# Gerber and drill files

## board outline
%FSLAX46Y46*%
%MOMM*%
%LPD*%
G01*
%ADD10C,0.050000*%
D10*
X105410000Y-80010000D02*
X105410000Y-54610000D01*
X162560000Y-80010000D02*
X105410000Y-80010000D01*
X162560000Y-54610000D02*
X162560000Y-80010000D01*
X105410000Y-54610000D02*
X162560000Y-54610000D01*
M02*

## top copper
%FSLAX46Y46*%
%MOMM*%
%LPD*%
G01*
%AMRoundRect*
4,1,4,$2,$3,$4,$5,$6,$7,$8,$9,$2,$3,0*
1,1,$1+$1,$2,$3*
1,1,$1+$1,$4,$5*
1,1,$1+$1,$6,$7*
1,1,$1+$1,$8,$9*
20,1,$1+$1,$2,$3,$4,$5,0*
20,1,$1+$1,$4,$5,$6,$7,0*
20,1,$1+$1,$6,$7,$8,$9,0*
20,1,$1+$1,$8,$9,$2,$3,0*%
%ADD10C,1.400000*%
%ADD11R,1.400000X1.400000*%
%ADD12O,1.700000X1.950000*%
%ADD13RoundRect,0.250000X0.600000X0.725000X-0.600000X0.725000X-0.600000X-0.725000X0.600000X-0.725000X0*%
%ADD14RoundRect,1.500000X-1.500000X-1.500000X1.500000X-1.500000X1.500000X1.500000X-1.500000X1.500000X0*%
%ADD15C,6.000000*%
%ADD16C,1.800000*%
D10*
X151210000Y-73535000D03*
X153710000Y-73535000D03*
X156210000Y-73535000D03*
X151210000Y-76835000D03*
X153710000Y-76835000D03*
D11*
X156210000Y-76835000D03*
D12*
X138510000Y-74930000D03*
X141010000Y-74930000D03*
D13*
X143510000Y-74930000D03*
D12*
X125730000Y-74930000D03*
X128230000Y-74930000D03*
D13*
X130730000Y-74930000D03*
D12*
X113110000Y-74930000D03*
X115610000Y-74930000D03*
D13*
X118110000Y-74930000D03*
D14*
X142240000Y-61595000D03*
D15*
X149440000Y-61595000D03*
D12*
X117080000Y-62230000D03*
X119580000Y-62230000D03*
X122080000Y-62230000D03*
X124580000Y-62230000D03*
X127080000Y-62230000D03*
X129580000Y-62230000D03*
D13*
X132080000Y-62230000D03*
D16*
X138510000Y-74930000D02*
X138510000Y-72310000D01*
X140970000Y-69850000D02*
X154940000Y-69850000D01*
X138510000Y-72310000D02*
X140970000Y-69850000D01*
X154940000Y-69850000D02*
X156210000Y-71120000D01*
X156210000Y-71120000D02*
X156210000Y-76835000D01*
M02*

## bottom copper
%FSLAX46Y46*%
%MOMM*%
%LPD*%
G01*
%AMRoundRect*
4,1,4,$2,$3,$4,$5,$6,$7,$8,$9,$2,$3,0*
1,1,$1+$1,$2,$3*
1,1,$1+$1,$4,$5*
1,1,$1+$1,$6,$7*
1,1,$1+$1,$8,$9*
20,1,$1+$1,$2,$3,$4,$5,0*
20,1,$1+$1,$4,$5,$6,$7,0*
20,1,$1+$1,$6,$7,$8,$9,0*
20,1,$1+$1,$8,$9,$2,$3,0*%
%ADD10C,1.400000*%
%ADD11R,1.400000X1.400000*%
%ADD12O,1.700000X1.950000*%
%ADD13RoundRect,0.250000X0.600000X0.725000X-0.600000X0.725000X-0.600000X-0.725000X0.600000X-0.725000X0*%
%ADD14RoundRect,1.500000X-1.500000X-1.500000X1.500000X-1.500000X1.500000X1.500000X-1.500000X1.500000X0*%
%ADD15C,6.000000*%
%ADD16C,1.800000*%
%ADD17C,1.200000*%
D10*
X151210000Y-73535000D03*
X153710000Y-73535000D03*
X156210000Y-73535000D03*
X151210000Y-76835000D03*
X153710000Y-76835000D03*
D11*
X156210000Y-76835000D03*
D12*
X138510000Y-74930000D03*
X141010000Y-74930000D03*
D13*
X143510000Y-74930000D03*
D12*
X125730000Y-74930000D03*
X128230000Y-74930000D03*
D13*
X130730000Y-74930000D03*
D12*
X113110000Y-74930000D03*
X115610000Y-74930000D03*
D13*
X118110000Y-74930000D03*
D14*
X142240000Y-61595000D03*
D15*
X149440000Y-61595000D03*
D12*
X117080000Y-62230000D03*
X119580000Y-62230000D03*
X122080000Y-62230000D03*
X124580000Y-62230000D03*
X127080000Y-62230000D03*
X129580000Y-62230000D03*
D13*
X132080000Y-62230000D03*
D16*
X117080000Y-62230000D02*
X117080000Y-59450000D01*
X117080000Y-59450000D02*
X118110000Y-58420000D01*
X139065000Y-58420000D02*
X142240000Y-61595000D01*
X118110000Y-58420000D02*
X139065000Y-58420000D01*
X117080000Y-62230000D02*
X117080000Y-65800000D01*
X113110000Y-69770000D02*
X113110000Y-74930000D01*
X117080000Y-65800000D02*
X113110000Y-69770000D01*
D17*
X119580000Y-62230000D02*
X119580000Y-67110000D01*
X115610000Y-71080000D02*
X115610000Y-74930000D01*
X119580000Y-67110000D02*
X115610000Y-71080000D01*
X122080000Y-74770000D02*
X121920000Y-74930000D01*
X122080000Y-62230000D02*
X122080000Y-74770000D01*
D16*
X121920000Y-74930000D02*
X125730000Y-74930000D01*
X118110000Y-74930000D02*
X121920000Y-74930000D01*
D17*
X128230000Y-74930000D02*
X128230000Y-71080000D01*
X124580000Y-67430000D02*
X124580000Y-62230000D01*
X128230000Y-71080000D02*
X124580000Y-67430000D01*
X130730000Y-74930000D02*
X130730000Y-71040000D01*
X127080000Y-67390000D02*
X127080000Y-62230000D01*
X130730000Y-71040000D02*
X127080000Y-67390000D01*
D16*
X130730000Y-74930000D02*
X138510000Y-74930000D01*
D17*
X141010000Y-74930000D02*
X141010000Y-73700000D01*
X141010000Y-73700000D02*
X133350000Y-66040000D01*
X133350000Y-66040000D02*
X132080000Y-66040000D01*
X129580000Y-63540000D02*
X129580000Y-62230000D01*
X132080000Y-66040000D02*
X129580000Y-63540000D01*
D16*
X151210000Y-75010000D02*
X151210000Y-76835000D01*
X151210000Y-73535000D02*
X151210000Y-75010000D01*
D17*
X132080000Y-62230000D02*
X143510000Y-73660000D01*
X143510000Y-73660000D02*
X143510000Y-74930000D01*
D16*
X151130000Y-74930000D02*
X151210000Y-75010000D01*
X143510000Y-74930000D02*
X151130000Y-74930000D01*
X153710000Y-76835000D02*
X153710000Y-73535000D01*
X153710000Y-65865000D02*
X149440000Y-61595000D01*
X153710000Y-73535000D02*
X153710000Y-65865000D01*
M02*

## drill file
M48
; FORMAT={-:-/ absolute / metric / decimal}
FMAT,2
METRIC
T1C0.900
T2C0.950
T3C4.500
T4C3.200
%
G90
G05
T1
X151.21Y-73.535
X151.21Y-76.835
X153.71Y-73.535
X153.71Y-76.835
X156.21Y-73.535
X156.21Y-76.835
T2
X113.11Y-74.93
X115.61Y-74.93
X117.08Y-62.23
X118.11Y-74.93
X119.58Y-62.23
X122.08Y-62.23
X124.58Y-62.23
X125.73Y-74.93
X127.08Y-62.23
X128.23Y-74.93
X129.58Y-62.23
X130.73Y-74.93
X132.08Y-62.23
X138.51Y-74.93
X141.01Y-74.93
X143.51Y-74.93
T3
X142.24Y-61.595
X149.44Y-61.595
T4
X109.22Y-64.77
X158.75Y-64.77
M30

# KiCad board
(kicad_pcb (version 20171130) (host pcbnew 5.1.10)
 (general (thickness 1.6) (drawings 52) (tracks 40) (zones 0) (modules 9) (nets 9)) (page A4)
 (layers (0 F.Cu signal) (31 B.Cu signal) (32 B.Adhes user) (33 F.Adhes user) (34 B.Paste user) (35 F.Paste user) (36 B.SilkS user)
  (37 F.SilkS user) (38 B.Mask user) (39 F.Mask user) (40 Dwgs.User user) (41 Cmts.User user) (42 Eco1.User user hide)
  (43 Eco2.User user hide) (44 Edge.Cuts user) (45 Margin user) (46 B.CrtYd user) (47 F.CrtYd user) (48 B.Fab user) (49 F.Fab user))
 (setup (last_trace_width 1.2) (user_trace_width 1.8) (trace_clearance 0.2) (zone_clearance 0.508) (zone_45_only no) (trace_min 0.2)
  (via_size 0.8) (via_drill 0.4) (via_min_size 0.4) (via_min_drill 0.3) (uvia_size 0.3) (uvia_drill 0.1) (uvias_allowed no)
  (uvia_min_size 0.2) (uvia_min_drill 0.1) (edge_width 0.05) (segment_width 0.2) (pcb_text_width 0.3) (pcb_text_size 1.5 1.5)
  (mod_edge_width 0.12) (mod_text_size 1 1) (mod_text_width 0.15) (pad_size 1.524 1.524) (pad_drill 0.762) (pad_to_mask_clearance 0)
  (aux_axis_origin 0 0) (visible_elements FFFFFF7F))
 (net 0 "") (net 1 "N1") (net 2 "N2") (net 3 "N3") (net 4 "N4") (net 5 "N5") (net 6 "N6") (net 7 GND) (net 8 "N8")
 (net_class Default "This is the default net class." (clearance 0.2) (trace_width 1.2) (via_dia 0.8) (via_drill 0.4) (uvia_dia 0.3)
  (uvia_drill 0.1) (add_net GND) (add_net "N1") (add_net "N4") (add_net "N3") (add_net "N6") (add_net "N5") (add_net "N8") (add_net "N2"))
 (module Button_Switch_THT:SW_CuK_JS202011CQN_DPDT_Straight (layer F.Cu) (at 156.21 76.835 180)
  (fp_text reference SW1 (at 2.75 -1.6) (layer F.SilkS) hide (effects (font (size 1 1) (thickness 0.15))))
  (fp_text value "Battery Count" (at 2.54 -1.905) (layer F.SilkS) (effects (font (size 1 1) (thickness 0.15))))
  (pad 6 thru_hole circle (at 5 3.3 180) (size 1.4 1.4) (drill 0.9) (layers *.Cu *.Mask) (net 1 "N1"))
  (pad 5 thru_hole circle (at 2.5 3.3 180) (size 1.4 1.4) (drill 0.9) (layers *.Cu *.Mask) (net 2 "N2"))
  (pad 4 thru_hole circle (at 0 3.3 180) (size 1.4 1.4) (drill 0.9) (layers *.Cu *.Mask) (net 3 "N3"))
  (pad 3 thru_hole circle (at 5 0 180) (size 1.4 1.4) (drill 0.9) (layers *.Cu *.Mask) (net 1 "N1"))
  (pad 2 thru_hole circle (at 2.5 0 180) (size 1.4 1.4) (drill 0.9) (layers *.Cu *.Mask) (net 2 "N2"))
  (pad 1 thru_hole rect (at 0 0 180) (size 1.4 1.4) (drill 0.9) (layers *.Cu *.Mask) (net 3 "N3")))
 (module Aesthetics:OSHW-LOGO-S (layer F.Cu) (at 109.22 58.42)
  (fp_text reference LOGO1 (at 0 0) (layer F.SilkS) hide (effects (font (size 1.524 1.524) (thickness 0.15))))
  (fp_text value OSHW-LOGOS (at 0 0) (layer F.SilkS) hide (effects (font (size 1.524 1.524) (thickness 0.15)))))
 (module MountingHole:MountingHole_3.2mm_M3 (layer F.Cu) (at 158.75 64.77)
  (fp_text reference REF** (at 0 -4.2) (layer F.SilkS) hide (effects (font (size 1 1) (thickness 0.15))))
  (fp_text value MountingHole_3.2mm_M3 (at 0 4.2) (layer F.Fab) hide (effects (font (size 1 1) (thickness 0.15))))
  (pad 1 np_thru_hole circle (at 0 0) (size 3.2 3.2) (drill 3.2) (layers *.Cu *.Mask)))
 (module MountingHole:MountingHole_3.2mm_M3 (layer F.Cu) (at 109.22 64.77)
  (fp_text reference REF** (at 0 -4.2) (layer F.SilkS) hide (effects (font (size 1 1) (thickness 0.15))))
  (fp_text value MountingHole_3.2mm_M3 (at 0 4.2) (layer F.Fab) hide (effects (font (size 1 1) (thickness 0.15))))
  (pad 1 np_thru_hole circle (at 0 0) (size 3.2 3.2) (drill 3.2) (layers *.Cu *.Mask)))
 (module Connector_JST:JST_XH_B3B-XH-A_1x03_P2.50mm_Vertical (layer F.Cu) (at 143.51 74.93 180)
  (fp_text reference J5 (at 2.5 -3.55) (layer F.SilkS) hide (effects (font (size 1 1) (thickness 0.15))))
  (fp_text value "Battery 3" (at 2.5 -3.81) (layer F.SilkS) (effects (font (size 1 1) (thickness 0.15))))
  (pad 3 thru_hole oval (at 5 0 180) (size 1.7 1.95) (drill 0.95) (layers *.Cu *.Mask) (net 3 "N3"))
  (pad 2 thru_hole oval (at 2.5 0 180) (size 1.7 1.95) (drill 0.95) (layers *.Cu *.Mask) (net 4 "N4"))
  (pad 1 thru_hole roundrect (at 0 0 180) (size 1.7 1.95) (drill 0.95) (layers *.Cu *.Mask) (roundrect_rratio 0.1470588235294118)
   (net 1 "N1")))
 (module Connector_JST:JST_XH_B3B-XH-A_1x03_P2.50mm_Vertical (layer F.Cu) (at 130.73 74.93 180)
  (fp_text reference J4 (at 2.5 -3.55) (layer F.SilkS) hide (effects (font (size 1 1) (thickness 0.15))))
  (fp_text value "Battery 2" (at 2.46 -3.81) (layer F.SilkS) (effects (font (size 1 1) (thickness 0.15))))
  (pad 3 thru_hole oval (at 5 0 180) (size 1.7 1.95) (drill 0.95) (layers *.Cu *.Mask) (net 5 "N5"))
  (pad 2 thru_hole oval (at 2.5 0 180) (size 1.7 1.95) (drill 0.95) (layers *.Cu *.Mask) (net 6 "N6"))
  (pad 1 thru_hole roundrect (at 0 0 180) (size 1.7 1.95) (drill 0.95) (layers *.Cu *.Mask) (roundrect_rratio 0.1470588235294118)
   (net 3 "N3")))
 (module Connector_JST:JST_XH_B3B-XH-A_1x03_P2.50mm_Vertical (layer F.Cu) (at 118.11 74.93 180)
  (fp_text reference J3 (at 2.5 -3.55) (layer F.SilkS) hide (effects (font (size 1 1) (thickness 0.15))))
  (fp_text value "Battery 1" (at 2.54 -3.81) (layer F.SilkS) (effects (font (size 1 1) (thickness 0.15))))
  (pad 3 thru_hole oval (at 5 0 180) (size 1.7 1.95) (drill 0.95) (layers *.Cu *.Mask) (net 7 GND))
  (pad 2 thru_hole oval (at 2.5 0 180) (size 1.7 1.95) (drill 0.95) (layers *.Cu *.Mask) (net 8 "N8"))
  (pad 1 thru_hole roundrect (at 0 0 180) (size 1.7 1.95) (drill 0.95) (layers *.Cu *.Mask) (roundrect_rratio 0.1470588235294118)
   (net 5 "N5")))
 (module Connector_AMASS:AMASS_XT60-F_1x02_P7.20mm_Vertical (layer F.Cu) (at 142.24 61.595)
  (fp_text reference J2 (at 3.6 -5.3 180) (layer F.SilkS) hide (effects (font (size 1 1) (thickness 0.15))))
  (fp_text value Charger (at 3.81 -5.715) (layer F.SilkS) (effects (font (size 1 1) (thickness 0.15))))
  (pad 1 thru_hole roundrect (at 0 0) (size 6 6) (drill 4.5) (layers *.Cu *.Mask) (roundrect_rratio 0.25) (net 7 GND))
  (pad 2 thru_hole circle (at 7.2 0) (size 6 6) (drill 4.5) (layers *.Cu *.Mask) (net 2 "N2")))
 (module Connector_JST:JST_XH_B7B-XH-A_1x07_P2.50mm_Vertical (layer F.Cu) (at 132.08 62.23 180)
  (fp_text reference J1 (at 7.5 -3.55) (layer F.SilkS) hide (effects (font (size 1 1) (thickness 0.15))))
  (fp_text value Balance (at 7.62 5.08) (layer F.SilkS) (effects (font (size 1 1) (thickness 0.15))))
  (pad 7 thru_hole oval (at 15 0 180) (size 1.7 1.95) (drill 0.95) (layers *.Cu *.Mask) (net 7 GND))
  (pad 6 thru_hole oval (at 12.5 0 180) (size 1.7 1.95) (drill 0.95) (layers *.Cu *.Mask) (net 8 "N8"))
  (pad 5 thru_hole oval (at 10 0 180) (size 1.7 1.95) (drill 0.95) (layers *.Cu *.Mask) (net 5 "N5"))
  (pad 4 thru_hole oval (at 7.5 0 180) (size 1.7 1.95) (drill 0.95) (layers *.Cu *.Mask) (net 6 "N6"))
  (pad 3 thru_hole oval (at 5 0 180) (size 1.7 1.95) (drill 0.95) (layers *.Cu *.Mask) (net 3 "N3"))
  (pad 2 thru_hole oval (at 2.5 0 180) (size 1.7 1.95) (drill 0.95) (layers *.Cu *.Mask) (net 4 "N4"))
  (pad 1 thru_hole roundrect (at 0 0 180) (size 1.7 1.95) (drill 0.95) (layers *.Cu *.Mask) (roundrect_rratio 0.1470588235294118)
   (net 1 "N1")))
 (gr_line (start 105.41 80.01) (end 105.41 54.61) (layer Edge.Cuts) (width 0.05))
 (gr_line (start 162.56 80.01) (end 105.41 80.01) (layer Edge.Cuts) (width 0.05))
 (gr_line (start 162.56 54.61) (end 162.56 80.01) (layer Edge.Cuts) (width 0.05))
 (gr_line (start 105.41 54.61) (end 162.56 54.61) (layer Edge.Cuts) (width 0.05))
 (segment (start 117.08 62.23) (end 117.08 59.45) (width 1.8) (layer B.Cu) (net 7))
 (segment (start 117.08 59.45) (end 118.11 58.42) (width 1.8) (layer B.Cu) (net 7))
 (segment (start 139.065 58.42) (end 142.24 61.595) (width 1.8) (layer B.Cu) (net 7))
 (segment (start 118.11 58.42) (end 139.065 58.42) (width 1.8) (layer B.Cu) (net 7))
 (segment (start 117.08 62.23) (end 117.08 65.8) (width 1.8) (layer B.Cu) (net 7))
 (segment (start 113.11 69.77) (end 113.11 74.93) (width 1.8) (layer B.Cu) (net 7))
 (segment (start 117.08 65.8) (end 113.11 69.77) (width 1.8) (layer B.Cu) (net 7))
 (segment (start 119.58 62.23) (end 119.58 67.11) (width 1.2) (layer B.Cu) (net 8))
 (segment (start 115.61 71.08) (end 115.61 74.93) (width 1.2) (layer B.Cu) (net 8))
 (segment (start 119.58 67.11) (end 115.61 71.08) (width 1.2) (layer B.Cu) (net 8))
 (segment (start 122.08 74.77) (end 121.92 74.93) (width 1.2) (layer B.Cu) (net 5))
 (segment (start 122.08 62.23) (end 122.08 74.77) (width 1.2) (layer B.Cu) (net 5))
 (segment (start 121.92 74.93) (end 125.73 74.93) (width 1.8) (layer B.Cu) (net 5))
 (segment (start 118.11 74.93) (end 121.92 74.93) (width 1.8) (layer B.Cu) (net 5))
 (segment (start 128.23 74.93) (end 128.23 71.08) (width 1.2) (layer B.Cu) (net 6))
 (segment (start 124.58 67.43) (end 124.58 62.23) (width 1.2) (layer B.Cu) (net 6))
 (segment (start 128.23 71.08) (end 124.58 67.43) (width 1.2) (layer B.Cu) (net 6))
 (segment (start 130.73 74.93) (end 130.73 71.04) (width 1.2) (layer B.Cu) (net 3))
 (segment (start 127.08 67.39) (end 127.08 62.23) (width 1.2) (layer B.Cu) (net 3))
 (segment (start 130.73 71.04) (end 127.08 67.39) (width 1.2) (layer B.Cu) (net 3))
 (segment (start 130.73 74.93) (end 138.51 74.93) (width 1.8) (layer B.Cu) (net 3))
 (segment (start 138.51 74.93) (end 138.51 72.31) (width 1.8) (layer F.Cu) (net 3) (status 1000000))
 (segment (start 140.97 69.85) (end 154.94 69.85) (width 1.8) (layer F.Cu) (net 3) (status 1000000))
 (segment (start 138.51 72.31) (end 140.97 69.85) (width 1.8) (layer F.Cu) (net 3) (status 1000000))
 (segment (start 154.94 69.85) (end 156.21 71.12) (width 1.8) (layer F.Cu) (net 3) (status 1000000))
 (segment (start 156.21 71.12) (end 156.21 76.835) (width 1.8) (layer F.Cu) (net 3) (status 1000000))
 (segment (start 141.01 74.93) (end 141.01 73.7) (width 1.2) (layer B.Cu) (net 4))
 (segment (start 141.01 73.7) (end 133.35 66.04) (width 1.2) (layer B.Cu) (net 4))
 (segment (start 133.35 66.04) (end 132.08 66.04) (width 1.2) (layer B.Cu) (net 4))
 (segment (start 129.58 63.54) (end 129.58 62.23) (width 1.2) (layer B.Cu) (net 4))
 (segment (start 132.08 66.04) (end 129.58 63.54) (width 1.2) (layer B.Cu) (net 4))
 (segment (start 151.21 75.01) (end 151.21 76.835) (width 1.8) (layer B.Cu) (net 1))
 (segment (start 151.21 73.535) (end 151.21 75.01) (width 1.8) (layer B.Cu) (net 1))
 (segment (start 132.08 62.23) (end 143.51 73.66) (width 1.2) (layer B.Cu) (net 1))
 (segment (start 143.51 73.66) (end 143.51 74.93) (width 1.2) (layer B.Cu) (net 1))
 (segment (start 151.13 74.93) (end 151.21 75.01) (width 1.8) (layer B.Cu) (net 1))
 (segment (start 143.51 74.93) (end 151.13 74.93) (width 1.8) (layer B.Cu) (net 1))
 (segment (start 153.71 76.835) (end 153.71 73.535) (width 1.8) (layer B.Cu) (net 2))
 (segment (start 153.71 65.865) (end 149.44 61.595) (width 1.8) (layer B.Cu) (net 2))
 (segment (start 153.71 73.535) (end 153.71 65.865) (width 1.8) (layer B.Cu) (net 2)))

